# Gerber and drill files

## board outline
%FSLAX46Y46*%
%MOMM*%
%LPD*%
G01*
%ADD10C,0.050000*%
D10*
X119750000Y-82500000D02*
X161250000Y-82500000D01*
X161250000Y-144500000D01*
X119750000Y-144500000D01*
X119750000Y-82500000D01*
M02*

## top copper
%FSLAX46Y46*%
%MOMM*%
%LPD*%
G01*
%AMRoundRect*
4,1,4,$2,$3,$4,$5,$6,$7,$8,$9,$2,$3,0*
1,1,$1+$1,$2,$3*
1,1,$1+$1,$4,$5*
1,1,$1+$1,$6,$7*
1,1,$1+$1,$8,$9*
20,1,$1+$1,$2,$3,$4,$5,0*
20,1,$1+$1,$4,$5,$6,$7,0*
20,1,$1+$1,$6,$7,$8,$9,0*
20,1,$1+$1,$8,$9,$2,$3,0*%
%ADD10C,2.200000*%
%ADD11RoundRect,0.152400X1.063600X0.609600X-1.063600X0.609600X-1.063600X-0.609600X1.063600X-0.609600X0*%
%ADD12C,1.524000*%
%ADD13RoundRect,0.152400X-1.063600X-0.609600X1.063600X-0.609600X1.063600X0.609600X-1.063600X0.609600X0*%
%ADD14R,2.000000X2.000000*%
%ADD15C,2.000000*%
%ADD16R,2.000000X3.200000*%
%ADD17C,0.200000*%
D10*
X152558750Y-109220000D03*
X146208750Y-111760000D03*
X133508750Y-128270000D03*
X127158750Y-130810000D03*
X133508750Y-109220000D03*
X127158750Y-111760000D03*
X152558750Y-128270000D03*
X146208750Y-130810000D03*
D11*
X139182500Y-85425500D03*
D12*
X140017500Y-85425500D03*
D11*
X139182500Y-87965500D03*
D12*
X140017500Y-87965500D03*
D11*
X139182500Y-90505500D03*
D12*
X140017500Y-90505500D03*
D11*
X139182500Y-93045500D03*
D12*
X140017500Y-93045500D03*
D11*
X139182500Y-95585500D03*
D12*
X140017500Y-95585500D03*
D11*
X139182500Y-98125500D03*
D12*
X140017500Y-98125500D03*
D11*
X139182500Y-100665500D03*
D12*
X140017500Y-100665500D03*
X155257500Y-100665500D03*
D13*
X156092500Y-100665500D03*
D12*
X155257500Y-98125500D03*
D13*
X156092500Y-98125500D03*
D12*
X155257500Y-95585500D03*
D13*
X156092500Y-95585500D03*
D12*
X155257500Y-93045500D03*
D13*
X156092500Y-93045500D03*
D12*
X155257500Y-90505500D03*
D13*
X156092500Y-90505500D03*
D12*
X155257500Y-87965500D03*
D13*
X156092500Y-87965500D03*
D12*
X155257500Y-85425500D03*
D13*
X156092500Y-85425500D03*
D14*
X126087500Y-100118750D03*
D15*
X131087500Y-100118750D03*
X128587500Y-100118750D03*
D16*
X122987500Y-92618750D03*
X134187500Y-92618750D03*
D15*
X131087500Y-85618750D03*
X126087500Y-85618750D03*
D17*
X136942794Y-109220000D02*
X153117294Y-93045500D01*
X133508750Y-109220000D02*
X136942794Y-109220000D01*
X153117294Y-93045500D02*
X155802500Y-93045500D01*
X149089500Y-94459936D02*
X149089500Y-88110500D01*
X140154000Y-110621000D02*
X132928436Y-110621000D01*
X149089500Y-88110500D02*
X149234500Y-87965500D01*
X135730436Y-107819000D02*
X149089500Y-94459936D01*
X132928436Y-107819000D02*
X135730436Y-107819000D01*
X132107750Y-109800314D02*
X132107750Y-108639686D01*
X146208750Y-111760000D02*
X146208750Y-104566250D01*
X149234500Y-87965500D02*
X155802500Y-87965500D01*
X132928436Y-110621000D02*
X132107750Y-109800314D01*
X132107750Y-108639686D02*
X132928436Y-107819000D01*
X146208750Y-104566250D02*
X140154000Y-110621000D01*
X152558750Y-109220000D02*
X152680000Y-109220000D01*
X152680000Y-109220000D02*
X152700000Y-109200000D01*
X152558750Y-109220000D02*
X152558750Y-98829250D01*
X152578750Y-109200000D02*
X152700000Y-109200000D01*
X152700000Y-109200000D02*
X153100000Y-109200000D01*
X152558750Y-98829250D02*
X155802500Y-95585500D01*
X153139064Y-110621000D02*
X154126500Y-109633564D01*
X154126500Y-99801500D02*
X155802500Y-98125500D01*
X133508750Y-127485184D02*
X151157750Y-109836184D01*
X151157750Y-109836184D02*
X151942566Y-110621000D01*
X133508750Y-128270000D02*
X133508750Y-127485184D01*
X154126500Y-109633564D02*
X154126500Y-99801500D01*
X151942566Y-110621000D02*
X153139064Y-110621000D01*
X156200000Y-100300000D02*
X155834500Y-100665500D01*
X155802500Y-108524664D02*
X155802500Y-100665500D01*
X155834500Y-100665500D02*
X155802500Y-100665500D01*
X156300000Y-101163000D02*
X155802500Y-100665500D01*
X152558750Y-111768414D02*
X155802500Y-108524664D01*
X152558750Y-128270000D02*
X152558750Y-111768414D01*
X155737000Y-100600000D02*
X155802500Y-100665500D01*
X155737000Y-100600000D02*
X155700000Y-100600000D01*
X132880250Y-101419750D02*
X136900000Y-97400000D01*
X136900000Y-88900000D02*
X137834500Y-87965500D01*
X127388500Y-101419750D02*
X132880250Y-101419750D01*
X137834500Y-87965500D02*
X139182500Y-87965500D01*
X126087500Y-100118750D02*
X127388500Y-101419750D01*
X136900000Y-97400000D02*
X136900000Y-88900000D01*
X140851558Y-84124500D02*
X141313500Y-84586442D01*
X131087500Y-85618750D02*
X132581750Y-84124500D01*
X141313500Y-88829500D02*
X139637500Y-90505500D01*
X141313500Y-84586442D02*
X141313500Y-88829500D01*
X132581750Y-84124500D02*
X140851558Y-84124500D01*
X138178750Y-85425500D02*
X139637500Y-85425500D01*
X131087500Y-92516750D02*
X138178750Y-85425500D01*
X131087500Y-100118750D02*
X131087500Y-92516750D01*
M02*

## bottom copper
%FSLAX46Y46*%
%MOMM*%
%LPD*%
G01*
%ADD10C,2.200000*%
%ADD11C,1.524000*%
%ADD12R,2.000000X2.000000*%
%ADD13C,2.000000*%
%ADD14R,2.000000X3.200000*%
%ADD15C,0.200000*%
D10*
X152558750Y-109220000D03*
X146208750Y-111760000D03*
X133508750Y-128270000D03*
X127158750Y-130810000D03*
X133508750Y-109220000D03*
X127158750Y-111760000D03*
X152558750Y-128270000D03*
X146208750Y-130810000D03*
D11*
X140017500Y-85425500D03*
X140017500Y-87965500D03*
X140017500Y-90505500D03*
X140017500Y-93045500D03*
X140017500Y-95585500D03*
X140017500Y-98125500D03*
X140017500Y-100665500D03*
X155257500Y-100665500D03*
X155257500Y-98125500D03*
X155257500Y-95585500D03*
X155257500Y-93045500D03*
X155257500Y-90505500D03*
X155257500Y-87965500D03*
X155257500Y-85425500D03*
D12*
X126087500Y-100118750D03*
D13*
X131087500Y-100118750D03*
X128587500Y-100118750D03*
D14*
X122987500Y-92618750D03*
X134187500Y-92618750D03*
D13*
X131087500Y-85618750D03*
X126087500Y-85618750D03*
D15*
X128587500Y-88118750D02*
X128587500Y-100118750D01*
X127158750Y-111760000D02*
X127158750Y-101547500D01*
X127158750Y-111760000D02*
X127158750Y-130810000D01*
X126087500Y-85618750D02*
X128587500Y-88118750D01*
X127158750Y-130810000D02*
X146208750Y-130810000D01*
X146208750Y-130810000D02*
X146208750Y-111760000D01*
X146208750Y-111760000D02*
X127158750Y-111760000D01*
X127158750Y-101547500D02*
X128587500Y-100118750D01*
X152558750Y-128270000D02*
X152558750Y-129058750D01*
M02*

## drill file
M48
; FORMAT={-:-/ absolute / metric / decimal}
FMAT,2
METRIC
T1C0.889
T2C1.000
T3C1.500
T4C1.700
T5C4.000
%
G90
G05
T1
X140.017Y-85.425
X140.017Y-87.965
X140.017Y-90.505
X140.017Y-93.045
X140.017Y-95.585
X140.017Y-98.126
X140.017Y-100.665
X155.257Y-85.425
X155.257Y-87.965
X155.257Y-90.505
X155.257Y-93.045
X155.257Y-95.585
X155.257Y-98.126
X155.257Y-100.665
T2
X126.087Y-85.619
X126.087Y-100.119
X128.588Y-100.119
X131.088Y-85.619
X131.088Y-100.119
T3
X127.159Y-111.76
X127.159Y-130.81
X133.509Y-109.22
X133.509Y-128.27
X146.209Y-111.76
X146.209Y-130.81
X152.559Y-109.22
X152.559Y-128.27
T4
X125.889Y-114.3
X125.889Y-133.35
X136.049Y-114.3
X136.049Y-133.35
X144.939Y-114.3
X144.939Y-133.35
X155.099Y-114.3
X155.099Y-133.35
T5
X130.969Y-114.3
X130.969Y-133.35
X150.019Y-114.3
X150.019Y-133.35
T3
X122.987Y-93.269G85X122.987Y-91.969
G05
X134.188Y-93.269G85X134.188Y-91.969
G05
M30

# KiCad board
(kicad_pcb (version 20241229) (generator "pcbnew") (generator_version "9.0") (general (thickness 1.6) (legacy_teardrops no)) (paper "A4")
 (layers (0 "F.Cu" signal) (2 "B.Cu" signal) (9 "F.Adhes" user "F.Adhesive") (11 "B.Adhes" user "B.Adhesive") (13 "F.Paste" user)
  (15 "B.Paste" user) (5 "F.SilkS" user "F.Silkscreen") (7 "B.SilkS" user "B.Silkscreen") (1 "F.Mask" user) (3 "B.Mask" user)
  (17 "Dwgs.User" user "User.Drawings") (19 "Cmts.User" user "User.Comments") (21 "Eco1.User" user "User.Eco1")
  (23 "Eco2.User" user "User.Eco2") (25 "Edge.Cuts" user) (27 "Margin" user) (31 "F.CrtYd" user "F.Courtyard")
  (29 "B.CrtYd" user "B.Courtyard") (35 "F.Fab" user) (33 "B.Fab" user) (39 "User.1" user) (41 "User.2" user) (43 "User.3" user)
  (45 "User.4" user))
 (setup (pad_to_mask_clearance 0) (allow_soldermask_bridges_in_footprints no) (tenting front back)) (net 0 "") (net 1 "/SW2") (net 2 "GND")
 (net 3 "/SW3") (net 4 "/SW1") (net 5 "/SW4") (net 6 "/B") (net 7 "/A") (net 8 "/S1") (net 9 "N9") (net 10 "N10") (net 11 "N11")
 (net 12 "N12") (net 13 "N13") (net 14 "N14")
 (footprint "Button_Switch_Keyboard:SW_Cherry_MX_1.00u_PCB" (layer "F.Cu") (at 152.55875 109.22)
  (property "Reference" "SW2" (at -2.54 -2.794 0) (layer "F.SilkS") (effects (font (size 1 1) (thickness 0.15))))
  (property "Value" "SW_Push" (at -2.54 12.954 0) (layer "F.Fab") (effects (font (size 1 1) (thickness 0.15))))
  (pad "" np_thru_hole circle (at -7.62 5.08) (size 1.7 1.7) (drill 1.7) (layers "*.Cu" "*.Mask"))
  (pad "" np_thru_hole circle (at -2.54 5.08) (size 4 4) (drill 4) (layers "*.Cu" "*.Mask"))
  (pad "" np_thru_hole circle (at 2.54 5.08) (size 1.7 1.7) (drill 1.7) (layers "*.Cu" "*.Mask"))
  (pad "1" thru_hole circle (at 0 0) (size 2.2 2.2) (drill 1.5) (layers "*.Cu" "*.Mask") (remove_unused_layers no) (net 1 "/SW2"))
  (pad "2" thru_hole circle (at -6.35 2.54) (size 2.2 2.2) (drill 1.5) (layers "*.Cu" "*.Mask") (remove_unused_layers no) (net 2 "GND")))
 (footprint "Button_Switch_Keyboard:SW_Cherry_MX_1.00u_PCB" (layer "F.Cu") (at 133.50875 128.27)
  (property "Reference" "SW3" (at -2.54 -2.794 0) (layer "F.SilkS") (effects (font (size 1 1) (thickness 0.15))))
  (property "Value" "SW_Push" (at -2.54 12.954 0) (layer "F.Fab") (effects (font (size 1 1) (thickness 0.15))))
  (pad "" np_thru_hole circle (at -7.62 5.08) (size 1.7 1.7) (drill 1.7) (layers "*.Cu" "*.Mask"))
  (pad "" np_thru_hole circle (at -2.54 5.08) (size 4 4) (drill 4) (layers "*.Cu" "*.Mask"))
  (pad "" np_thru_hole circle (at 2.54 5.08) (size 1.7 1.7) (drill 1.7) (layers "*.Cu" "*.Mask"))
  (pad "1" thru_hole circle (at 0 0) (size 2.2 2.2) (drill 1.5) (layers "*.Cu" "*.Mask") (remove_unused_layers no) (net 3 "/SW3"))
  (pad "2" thru_hole circle (at -6.35 2.54) (size 2.2 2.2) (drill 1.5) (layers "*.Cu" "*.Mask") (remove_unused_layers no) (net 2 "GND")))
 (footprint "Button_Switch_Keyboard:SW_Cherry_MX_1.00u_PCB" (layer "F.Cu") (at 133.50875 109.22)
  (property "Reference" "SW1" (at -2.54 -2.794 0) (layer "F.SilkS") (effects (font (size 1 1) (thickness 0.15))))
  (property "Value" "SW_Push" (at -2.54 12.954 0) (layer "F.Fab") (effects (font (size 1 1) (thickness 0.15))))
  (pad "" np_thru_hole circle (at -7.62 5.08) (size 1.7 1.7) (drill 1.7) (layers "*.Cu" "*.Mask"))
  (pad "" np_thru_hole circle (at -2.54 5.08) (size 4 4) (drill 4) (layers "*.Cu" "*.Mask"))
  (pad "" np_thru_hole circle (at 2.54 5.08) (size 1.7 1.7) (drill 1.7) (layers "*.Cu" "*.Mask"))
  (pad "1" thru_hole circle (at 0 0) (size 2.2 2.2) (drill 1.5) (layers "*.Cu" "*.Mask") (remove_unused_layers no) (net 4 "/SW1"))
  (pad "2" thru_hole circle (at -6.35 2.54) (size 2.2 2.2) (drill 1.5) (layers "*.Cu" "*.Mask") (remove_unused_layers no) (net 2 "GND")))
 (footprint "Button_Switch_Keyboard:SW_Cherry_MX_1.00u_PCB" (layer "F.Cu") (at 152.55875 128.27)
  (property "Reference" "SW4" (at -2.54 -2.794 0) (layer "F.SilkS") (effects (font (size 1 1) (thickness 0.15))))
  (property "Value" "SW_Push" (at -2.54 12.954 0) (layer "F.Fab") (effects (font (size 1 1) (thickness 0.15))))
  (pad "" np_thru_hole circle (at -7.62 5.08) (size 1.7 1.7) (drill 1.7) (layers "*.Cu" "*.Mask"))
  (pad "" np_thru_hole circle (at -2.54 5.08) (size 4 4) (drill 4) (layers "*.Cu" "*.Mask"))
  (pad "" np_thru_hole circle (at 2.54 5.08) (size 1.7 1.7) (drill 1.7) (layers "*.Cu" "*.Mask"))
  (pad "1" thru_hole circle (at 0 0) (size 2.2 2.2) (drill 1.5) (layers "*.Cu" "*.Mask") (remove_unused_layers no) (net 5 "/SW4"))
  (pad "2" thru_hole circle (at -6.35 2.54) (size 2.2 2.2) (drill 1.5) (layers "*.Cu" "*.Mask") (remove_unused_layers no) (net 2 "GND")))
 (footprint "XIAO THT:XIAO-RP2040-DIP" (layer "F.Cu") (at 147.6375 93.0455)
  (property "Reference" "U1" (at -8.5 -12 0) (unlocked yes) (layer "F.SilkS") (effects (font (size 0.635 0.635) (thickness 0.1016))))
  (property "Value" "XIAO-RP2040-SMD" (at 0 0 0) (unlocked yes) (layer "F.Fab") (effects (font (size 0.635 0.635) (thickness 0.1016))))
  (pad "1" smd roundrect (at -8.455 -7.62 180) (size 2.432 1.524) (layers "F.Cu" "F.Mask") (roundrect_rratio 0.1) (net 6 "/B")
   (thermal_bridge_angle 45))
  (pad "1" thru_hole circle (at -7.62 -7.62 180) (size 1.524 1.524) (drill 0.889) (layers "*.Cu" "*.Mask") (remove_unused_layers no)
   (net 6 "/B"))
  (pad "2" smd roundrect (at -8.455 -5.08 180) (size 2.432 1.524) (layers "F.Cu" "F.Mask") (roundrect_rratio 0.1) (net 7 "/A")
   (thermal_bridge_angle 45))
  (pad "2" thru_hole circle (at -7.62 -5.08 180) (size 1.524 1.524) (drill 0.889) (layers "*.Cu" "*.Mask") (remove_unused_layers no)
   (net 7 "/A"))
  (pad "3" smd roundrect (at -8.455 -2.54 180) (size 2.432 1.524) (layers "F.Cu" "F.Mask") (roundrect_rratio 0.1) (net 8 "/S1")
   (thermal_bridge_angle 45))
  (pad "3" thru_hole circle (at -7.62 -2.54 180) (size 1.524 1.524) (drill 0.889) (layers "*.Cu" "*.Mask") (remove_unused_layers no)
   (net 8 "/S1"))
  (pad "4" smd roundrect (at -8.455 0 180) (size 2.432 1.524) (layers "F.Cu" "F.Mask") (roundrect_rratio 0.1) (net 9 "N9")
   (thermal_bridge_angle 45))
  (pad "4" thru_hole circle (at -7.62 0 180) (size 1.524 1.524) (drill 0.889) (layers "*.Cu" "*.Mask") (remove_unused_layers no)
   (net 9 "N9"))
  (pad "5" smd roundrect (at -8.455 2.54 180) (size 2.432 1.524) (layers "F.Cu" "F.Mask") (roundrect_rratio 0.1) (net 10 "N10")
   (thermal_bridge_angle 45))
  (pad "5" thru_hole circle (at -7.62 2.54 180) (size 1.524 1.524) (drill 0.889) (layers "*.Cu" "*.Mask") (remove_unused_layers no)
   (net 10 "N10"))
  (pad "6" smd roundrect (at -8.455 5.08 180) (size 2.432 1.524) (layers "F.Cu" "F.Mask") (roundrect_rratio 0.1) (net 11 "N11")
   (thermal_bridge_angle 45))
  (pad "6" thru_hole circle (at -7.62 5.08 180) (size 1.524 1.524) (drill 0.889) (layers "*.Cu" "*.Mask") (remove_unused_layers no)
   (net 11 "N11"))
  (pad "7" smd roundrect (at -8.455 7.62 180) (size 2.432 1.524) (layers "F.Cu" "F.Mask") (roundrect_rratio 0.1) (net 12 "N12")
   (thermal_bridge_angle 45))
  (pad "7" thru_hole circle (at -7.62 7.62 180) (size 1.524 1.524) (drill 0.889) (layers "*.Cu" "*.Mask") (remove_unused_layers no)
   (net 12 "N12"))
  (pad "8" thru_hole circle (at 7.62 7.62) (size 1.524 1.524) (drill 0.889) (layers "*.Cu" "*.Mask") (remove_unused_layers no)
   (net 5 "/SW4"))
  (pad "8" smd roundrect (at 8.455 7.62) (size 2.432 1.524) (layers "F.Cu" "F.Mask") (roundrect_rratio 0.1) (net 5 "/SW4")
   (thermal_bridge_angle 45))
  (pad "9" thru_hole circle (at 7.62 5.08) (size 1.524 1.524) (drill 0.889) (layers "*.Cu" "*.Mask") (remove_unused_layers no)
   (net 3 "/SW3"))
  (pad "9" smd roundrect (at 8.455 5.08) (size 2.432 1.524) (layers "F.Cu" "F.Mask") (roundrect_rratio 0.1) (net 3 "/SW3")
   (thermal_bridge_angle 45))
  (pad "10" thru_hole circle (at 7.62 2.54) (size 1.524 1.524) (drill 0.889) (layers "*.Cu" "*.Mask") (remove_unused_layers no)
   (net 1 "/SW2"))
  (pad "10" smd roundrect (at 8.455 2.54) (size 2.432 1.524) (layers "F.Cu" "F.Mask") (roundrect_rratio 0.1) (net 1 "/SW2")
   (thermal_bridge_angle 45))
  (pad "11" thru_hole circle (at 7.62 0) (size 1.524 1.524) (drill 0.889) (layers "*.Cu" "*.Mask") (remove_unused_layers no) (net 4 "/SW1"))
  (pad "11" smd roundrect (at 8.455 0) (size 2.432 1.524) (layers "F.Cu" "F.Mask") (roundrect_rratio 0.1) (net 4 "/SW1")
   (thermal_bridge_angle 45))
  (pad "12" thru_hole circle (at 7.62 -2.54) (size 1.524 1.524) (drill 0.889) (layers "*.Cu" "*.Mask") (remove_unused_layers no)
   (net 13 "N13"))
  (pad "12" smd roundrect (at 8.455 -2.54) (size 2.432 1.524) (layers "F.Cu" "F.Mask") (roundrect_rratio 0.1) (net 13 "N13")
   (thermal_bridge_angle 45))
  (pad "13" thru_hole circle (at 7.62 -5.08) (size 1.524 1.524) (drill 0.889) (layers "*.Cu" "*.Mask") (remove_unused_layers no)
   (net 2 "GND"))
  (pad "13" smd roundrect (at 8.455 -5.08) (size 2.432 1.524) (layers "F.Cu" "F.Mask") (roundrect_rratio 0.1) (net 2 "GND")
   (thermal_bridge_angle 45))
  (pad "14" thru_hole circle (at 7.62 -7.62) (size 1.524 1.524) (drill 0.889) (layers "*.Cu" "*.Mask") (remove_unused_layers no)
   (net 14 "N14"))
  (pad "14" smd roundrect (at 8.455 -7.62) (size 2.432 1.524) (layers "F.Cu" "F.Mask") (roundrect_rratio 0.1) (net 14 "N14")
   (thermal_bridge_angle 45)))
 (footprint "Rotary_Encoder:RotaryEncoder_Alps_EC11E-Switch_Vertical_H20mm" (layer "F.Cu") (at 126.0875 100.11875 90)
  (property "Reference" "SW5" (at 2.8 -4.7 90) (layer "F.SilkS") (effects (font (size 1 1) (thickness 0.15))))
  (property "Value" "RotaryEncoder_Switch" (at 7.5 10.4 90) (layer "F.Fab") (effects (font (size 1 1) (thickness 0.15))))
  (pad "A" thru_hole rect (at 0 0 90) (size 2 2) (drill 1) (layers "*.Cu" "*.Mask") (remove_unused_layers no) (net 7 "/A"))
  (pad "B" thru_hole circle (at 0 5 90) (size 2 2) (drill 1) (layers "*.Cu" "*.Mask") (remove_unused_layers no) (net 6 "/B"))
  (pad "C" thru_hole circle (at 0 2.5 90) (size 2 2) (drill 1) (layers "*.Cu" "*.Mask") (remove_unused_layers no) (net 2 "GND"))
  (pad "MP" thru_hole rect (at 7.5 -3.1 90) (size 3.2 2) (drill oval 2.8 1.5) (layers "*.Cu" "*.Mask") (remove_unused_layers no))
  (pad "MP" thru_hole rect (at 7.5 8.1 90) (size 3.2 2) (drill oval 2.8 1.5) (layers "*.Cu" "*.Mask") (remove_unused_layers no))
  (pad "S1" thru_hole circle (at 14.5 5 90) (size 2 2) (drill 1) (layers "*.Cu" "*.Mask") (remove_unused_layers no) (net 8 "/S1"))
  (pad "S2" thru_hole circle (at 14.5 0 90) (size 2 2) (drill 1) (layers "*.Cu" "*.Mask") (remove_unused_layers no) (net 2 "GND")))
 (gr_rect (start 119.75 82.5) (end 161.25 144.5) (stroke (width 0.05) (type default)) (fill no) (layer "Edge.Cuts"))
 (segment (start 136.942794 109.22) (end 153.117294 93.0455) (width 0.2) (layer "F.Cu") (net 4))
 (segment (start 133.50875 109.22) (end 136.942794 109.22) (width 0.2) (layer "F.Cu") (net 4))
 (segment (start 153.117294 93.0455) (end 155.8025 93.0455) (width 0.2) (layer "F.Cu") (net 4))
 (segment (start 149.0895 94.459936) (end 149.0895 88.1105) (width 0.2) (layer "F.Cu") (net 2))
 (segment (start 140.154 110.621) (end 132.928436 110.621) (width 0.2) (layer "F.Cu") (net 2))
 (segment (start 149.0895 88.1105) (end 149.2345 87.9655) (width 0.2) (layer "F.Cu") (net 2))
 (segment (start 135.730436 107.819) (end 149.0895 94.459936) (width 0.2) (layer "F.Cu") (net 2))
 (segment (start 132.928436 107.819) (end 135.730436 107.819) (width 0.2) (layer "F.Cu") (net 2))
 (segment (start 132.10775 109.800314) (end 132.10775 108.639686) (width 0.2) (layer "F.Cu") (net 2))
 (segment (start 146.20875 111.76) (end 146.20875 104.56625) (width 0.2) (layer "F.Cu") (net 2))
 (segment (start 149.2345 87.9655) (end 155.8025 87.9655) (width 0.2) (layer "F.Cu") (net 2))
 (segment (start 132.928436 110.621) (end 132.10775 109.800314) (width 0.2) (layer "F.Cu") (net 2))
 (segment (start 132.10775 108.639686) (end 132.928436 107.819) (width 0.2) (layer "F.Cu") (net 2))
 (segment (start 146.20875 104.56625) (end 140.154 110.621) (width 0.2) (layer "F.Cu") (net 2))
 (segment (start 128.5875 88.11875) (end 128.5875 100.11875) (width 0.2) (layer "B.Cu") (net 2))
 (segment (start 127.15875 111.76) (end 127.15875 101.5475) (width 0.2) (layer "B.Cu") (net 2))
 (segment (start 127.15875 111.76) (end 127.15875 130.81) (width 0.2) (layer "B.Cu") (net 2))
 (segment (start 126.0875 85.61875) (end 128.5875 88.11875) (width 0.2) (layer "B.Cu") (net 2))
 (segment (start 127.15875 130.81) (end 146.20875 130.81) (width 0.2) (layer "B.Cu") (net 2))
 (segment (start 146.20875 130.81) (end 146.20875 111.76) (width 0.2) (layer "B.Cu") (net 2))
 (segment (start 146.20875 111.76) (end 127.15875 111.76) (width 0.2) (layer "B.Cu") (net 2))
 (segment (start 127.15875 101.5475) (end 128.5875 100.11875) (width 0.2) (layer "B.Cu") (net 2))
 (segment (start 152.55875 109.22) (end 152.68 109.22) (width 0.2) (layer "F.Cu") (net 1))
 (segment (start 152.68 109.22) (end 152.7 109.2) (width 0.2) (layer "F.Cu") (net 1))
 (segment (start 152.55875 109.22) (end 152.55875 98.82925) (width 0.2) (layer "F.Cu") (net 1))
 (segment (start 152.57875 109.2) (end 152.7 109.2) (width 0.2) (layer "F.Cu") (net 1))
 (segment (start 152.7 109.2) (end 153.1 109.2) (width 0.2) (layer "F.Cu") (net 1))
 (segment (start 152.55875 98.82925) (end 155.8025 95.5855) (width 0.2) (layer "F.Cu") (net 1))
 (segment (start 153.139064 110.621) (end 154.1265 109.633564) (width 0.2) (layer "F.Cu") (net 3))
 (segment (start 154.1265 99.8015) (end 155.8025 98.1255) (width 0.2) (layer "F.Cu") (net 3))
 (segment (start 133.50875 127.485184) (end 151.15775 109.836184) (width 0.2) (layer "F.Cu") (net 3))
 (segment (start 151.15775 109.836184) (end 151.942566 110.621) (width 0.2) (layer "F.Cu") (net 3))
 (segment (start 133.50875 128.27) (end 133.50875 127.485184) (width 0.2) (layer "F.Cu") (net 3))
 (segment (start 154.1265 109.633564) (end 154.1265 99.8015) (width 0.2) (layer "F.Cu") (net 3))
 (segment (start 151.942566 110.621) (end 153.139064 110.621) (width 0.2) (layer "F.Cu") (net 3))
 (segment (start 156.2 100.3) (end 155.8345 100.6655) (width 0.2) (layer "F.Cu") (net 5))
 (segment (start 155.8025 108.524664) (end 155.8025 100.6655) (width 0.2) (layer "F.Cu") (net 5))
 (segment (start 155.8345 100.6655) (end 155.8025 100.6655) (width 0.2) (layer "F.Cu") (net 5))
 (segment (start 156.3 101.163) (end 155.8025 100.6655) (width 0.2) (layer "F.Cu") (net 5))
 (segment (start 152.55875 111.768414) (end 155.8025 108.524664) (width 0.2) (layer "F.Cu") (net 5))
 (segment (start 152.55875 128.27) (end 152.55875 111.768414) (width 0.2) (layer "F.Cu") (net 5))
 (segment (start 155.737 100.6) (end 155.8025 100.6655) (width 0.2) (layer "F.Cu") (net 5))
 (segment (start 155.737 100.6) (end 155.7 100.6) (width 0.2) (layer "F.Cu") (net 5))
 (segment (start 152.55875 128.27) (end 152.55875 129.05875) (width 0.2) (layer "B.Cu") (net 5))
 (segment (start 132.88025 101.41975) (end 136.9 97.4) (width 0.2) (layer "F.Cu") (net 7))
 (segment (start 136.9 88.9) (end 137.8345 87.9655) (width 0.2) (layer "F.Cu") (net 7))
 (segment (start 127.3885 101.41975) (end 132.88025 101.41975) (width 0.2) (layer "F.Cu") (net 7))
 (segment (start 137.8345 87.9655) (end 139.1825 87.9655) (width 0.2) (layer "F.Cu") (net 7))
 (segment (start 126.0875 100.11875) (end 127.3885 101.41975) (width 0.2) (layer "F.Cu") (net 7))
 (segment (start 136.9 97.4) (end 136.9 88.9) (width 0.2) (layer "F.Cu") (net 7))
 (segment (start 140.851558 84.1245) (end 141.3135 84.586442) (width 0.2) (layer "F.Cu") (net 8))
 (segment (start 131.0875 85.61875) (end 132.58175 84.1245) (width 0.2) (layer "F.Cu") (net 8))
 (segment (start 141.3135 88.8295) (end 139.6375 90.5055) (width 0.2) (layer "F.Cu") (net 8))
 (segment (start 141.3135 84.586442) (end 141.3135 88.8295) (width 0.2) (layer "F.Cu") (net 8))
 (segment (start 132.58175 84.1245) (end 140.851558 84.1245) (width 0.2) (layer "F.Cu") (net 8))
 (segment (start 138.17875 85.4255) (end 139.6375 85.4255) (width 0.2) (layer "F.Cu") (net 6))
 (segment (start 131.0875 92.51675) (end 138.17875 85.4255) (width 0.2) (layer "F.Cu") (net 6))
 (segment (start 131.0875 100.11875) (end 131.0875 92.51675) (width 0.2) (layer "F.Cu") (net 6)))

